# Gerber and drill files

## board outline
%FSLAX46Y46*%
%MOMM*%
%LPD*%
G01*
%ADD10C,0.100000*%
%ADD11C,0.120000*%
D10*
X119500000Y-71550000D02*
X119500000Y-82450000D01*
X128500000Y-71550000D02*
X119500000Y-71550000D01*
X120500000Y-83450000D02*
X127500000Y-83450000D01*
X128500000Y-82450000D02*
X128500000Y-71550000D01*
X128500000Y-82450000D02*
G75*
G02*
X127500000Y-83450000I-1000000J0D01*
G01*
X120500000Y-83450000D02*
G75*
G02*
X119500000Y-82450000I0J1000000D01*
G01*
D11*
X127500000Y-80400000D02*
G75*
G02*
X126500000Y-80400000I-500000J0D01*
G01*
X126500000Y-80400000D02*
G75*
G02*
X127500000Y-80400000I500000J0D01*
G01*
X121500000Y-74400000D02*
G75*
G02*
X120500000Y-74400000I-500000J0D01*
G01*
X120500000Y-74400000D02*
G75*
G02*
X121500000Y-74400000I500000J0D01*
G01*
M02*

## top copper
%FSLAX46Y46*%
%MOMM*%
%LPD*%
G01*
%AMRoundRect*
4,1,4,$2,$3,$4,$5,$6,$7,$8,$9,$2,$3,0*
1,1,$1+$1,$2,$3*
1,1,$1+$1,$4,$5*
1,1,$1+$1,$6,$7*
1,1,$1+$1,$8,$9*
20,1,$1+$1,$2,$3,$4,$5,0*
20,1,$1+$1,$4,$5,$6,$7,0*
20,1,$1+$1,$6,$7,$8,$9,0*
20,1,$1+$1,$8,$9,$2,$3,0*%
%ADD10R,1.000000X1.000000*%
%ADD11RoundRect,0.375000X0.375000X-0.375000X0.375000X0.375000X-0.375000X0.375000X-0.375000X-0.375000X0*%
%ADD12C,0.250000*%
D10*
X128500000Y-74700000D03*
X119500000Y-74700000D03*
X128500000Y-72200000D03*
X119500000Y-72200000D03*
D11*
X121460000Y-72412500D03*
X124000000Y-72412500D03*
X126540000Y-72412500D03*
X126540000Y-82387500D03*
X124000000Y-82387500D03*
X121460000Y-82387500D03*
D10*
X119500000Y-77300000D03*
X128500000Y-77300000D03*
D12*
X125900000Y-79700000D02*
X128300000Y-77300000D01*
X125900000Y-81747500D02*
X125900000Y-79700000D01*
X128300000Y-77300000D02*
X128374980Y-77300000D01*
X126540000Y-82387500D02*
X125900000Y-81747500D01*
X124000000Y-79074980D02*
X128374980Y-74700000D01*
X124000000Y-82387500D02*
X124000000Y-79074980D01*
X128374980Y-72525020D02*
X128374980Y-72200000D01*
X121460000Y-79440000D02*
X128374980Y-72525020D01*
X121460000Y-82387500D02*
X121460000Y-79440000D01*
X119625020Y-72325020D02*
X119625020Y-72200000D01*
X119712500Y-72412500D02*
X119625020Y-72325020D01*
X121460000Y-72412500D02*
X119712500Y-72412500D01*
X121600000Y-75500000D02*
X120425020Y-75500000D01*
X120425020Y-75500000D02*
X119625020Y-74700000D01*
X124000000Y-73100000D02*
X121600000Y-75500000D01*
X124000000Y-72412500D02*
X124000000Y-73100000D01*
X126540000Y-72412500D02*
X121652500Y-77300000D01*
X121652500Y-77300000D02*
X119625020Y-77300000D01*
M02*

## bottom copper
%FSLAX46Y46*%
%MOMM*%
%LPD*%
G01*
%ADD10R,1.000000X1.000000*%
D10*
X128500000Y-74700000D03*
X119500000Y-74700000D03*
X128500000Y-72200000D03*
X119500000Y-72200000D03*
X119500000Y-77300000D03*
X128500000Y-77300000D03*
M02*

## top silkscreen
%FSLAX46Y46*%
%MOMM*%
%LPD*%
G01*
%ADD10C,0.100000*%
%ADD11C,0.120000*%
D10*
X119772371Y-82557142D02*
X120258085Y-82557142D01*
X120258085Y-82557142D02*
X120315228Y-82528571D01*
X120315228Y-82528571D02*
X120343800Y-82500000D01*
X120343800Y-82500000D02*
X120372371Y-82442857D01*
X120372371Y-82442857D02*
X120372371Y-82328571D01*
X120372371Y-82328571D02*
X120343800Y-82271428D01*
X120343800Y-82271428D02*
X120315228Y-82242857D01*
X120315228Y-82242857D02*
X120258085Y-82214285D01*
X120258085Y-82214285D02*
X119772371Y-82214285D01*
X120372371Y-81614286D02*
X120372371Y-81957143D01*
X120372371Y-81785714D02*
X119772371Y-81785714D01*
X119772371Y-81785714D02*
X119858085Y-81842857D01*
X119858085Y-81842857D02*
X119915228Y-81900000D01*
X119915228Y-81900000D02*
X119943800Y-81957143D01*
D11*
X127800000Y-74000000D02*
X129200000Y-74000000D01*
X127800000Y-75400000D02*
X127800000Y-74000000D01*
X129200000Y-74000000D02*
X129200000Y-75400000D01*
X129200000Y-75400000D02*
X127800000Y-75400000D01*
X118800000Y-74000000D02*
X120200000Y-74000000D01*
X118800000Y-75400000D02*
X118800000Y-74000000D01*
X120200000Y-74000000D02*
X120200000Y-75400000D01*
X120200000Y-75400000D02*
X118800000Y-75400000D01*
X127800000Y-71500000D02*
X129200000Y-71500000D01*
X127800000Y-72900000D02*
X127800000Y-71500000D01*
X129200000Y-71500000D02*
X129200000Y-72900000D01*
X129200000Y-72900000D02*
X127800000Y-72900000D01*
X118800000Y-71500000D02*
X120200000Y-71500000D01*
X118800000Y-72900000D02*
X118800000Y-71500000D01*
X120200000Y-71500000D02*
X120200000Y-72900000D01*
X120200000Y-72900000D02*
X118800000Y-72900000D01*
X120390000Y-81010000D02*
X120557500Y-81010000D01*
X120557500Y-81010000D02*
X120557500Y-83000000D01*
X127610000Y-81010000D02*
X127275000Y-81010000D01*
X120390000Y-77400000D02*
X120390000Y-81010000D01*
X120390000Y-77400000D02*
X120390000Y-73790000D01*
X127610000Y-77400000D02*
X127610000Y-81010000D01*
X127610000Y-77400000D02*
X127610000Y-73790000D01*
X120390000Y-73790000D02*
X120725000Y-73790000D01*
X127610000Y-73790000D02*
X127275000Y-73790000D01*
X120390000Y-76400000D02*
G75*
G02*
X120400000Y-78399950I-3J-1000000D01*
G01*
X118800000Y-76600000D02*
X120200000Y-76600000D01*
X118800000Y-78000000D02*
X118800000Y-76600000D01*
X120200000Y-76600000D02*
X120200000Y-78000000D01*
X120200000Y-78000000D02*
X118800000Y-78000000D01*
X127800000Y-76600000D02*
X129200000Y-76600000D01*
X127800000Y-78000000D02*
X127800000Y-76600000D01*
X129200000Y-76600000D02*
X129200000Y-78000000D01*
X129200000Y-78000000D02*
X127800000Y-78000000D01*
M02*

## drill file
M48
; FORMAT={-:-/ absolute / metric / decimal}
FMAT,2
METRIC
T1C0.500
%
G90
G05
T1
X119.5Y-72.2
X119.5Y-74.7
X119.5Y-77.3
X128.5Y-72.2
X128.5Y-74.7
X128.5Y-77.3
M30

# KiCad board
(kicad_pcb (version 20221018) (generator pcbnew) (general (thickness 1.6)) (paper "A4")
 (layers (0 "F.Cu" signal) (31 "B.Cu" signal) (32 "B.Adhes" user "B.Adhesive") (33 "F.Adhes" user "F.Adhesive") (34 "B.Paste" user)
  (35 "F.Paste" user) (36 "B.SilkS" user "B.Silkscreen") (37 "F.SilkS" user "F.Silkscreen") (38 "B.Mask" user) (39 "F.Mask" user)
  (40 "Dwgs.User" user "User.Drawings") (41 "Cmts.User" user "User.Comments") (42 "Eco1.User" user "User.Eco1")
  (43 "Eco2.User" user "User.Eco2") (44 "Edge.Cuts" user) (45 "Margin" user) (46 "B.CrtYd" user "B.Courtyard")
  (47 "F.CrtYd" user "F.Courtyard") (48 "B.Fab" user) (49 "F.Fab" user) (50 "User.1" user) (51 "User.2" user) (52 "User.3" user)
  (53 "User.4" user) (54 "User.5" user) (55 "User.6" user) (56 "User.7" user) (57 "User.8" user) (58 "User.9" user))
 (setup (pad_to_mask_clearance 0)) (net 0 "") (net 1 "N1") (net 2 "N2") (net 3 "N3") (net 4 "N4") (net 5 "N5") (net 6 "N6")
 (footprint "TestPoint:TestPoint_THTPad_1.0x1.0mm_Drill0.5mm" (layer "F.Cu") (at 128.5 74.7)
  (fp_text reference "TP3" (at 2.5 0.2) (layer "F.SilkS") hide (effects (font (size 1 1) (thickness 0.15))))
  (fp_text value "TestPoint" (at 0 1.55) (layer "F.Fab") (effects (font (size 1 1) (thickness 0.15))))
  (fp_line (start -0.7 -0.7) (end 0.7 -0.7) (stroke (width 0.12) (type solid)) (layer "F.SilkS"))
  (fp_line (start -0.7 0.7) (end -0.7 -0.7) (stroke (width 0.12) (type solid)) (layer "F.SilkS"))
  (fp_line (start 0.7 -0.7) (end 0.7 0.7) (stroke (width 0.12) (type solid)) (layer "F.SilkS"))
  (fp_line (start 0.7 0.7) (end -0.7 0.7) (stroke (width 0.12) (type solid)) (layer "F.SilkS"))
  (pad "1" thru_hole rect (at 0 0) (size 1 1) (drill 0.5) (layers "*.Cu" "*.Mask") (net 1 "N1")))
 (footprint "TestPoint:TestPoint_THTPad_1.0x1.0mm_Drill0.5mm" (layer "F.Cu") (at 119.5 74.7)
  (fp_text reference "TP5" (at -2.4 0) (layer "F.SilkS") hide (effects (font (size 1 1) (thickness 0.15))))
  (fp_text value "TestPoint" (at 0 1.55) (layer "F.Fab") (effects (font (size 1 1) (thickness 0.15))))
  (fp_line (start -0.7 -0.7) (end 0.7 -0.7) (stroke (width 0.12) (type solid)) (layer "F.SilkS"))
  (fp_line (start -0.7 0.7) (end -0.7 -0.7) (stroke (width 0.12) (type solid)) (layer "F.SilkS"))
  (fp_line (start 0.7 -0.7) (end 0.7 0.7) (stroke (width 0.12) (type solid)) (layer "F.SilkS"))
  (fp_line (start 0.7 0.7) (end -0.7 0.7) (stroke (width 0.12) (type solid)) (layer "F.SilkS"))
  (pad "1" thru_hole rect (at 0 0) (size 1 1) (drill 0.5) (layers "*.Cu" "*.Mask") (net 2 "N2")))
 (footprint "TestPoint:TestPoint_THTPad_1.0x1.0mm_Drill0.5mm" (layer "F.Cu") (at 128.5 72.2)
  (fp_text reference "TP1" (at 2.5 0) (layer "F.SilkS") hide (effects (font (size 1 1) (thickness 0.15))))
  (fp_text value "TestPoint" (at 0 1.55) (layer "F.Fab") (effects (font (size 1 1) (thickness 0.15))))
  (fp_line (start -0.7 -0.7) (end 0.7 -0.7) (stroke (width 0.12) (type solid)) (layer "F.SilkS"))
  (fp_line (start -0.7 0.7) (end -0.7 -0.7) (stroke (width 0.12) (type solid)) (layer "F.SilkS"))
  (fp_line (start 0.7 -0.7) (end 0.7 0.7) (stroke (width 0.12) (type solid)) (layer "F.SilkS"))
  (fp_line (start 0.7 0.7) (end -0.7 0.7) (stroke (width 0.12) (type solid)) (layer "F.SilkS"))
  (pad "1" thru_hole rect (at 0 0) (size 1 1) (drill 0.5) (layers "*.Cu" "*.Mask") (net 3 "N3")))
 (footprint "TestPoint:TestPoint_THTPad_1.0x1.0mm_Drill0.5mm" (layer "F.Cu") (at 119.5 72.2)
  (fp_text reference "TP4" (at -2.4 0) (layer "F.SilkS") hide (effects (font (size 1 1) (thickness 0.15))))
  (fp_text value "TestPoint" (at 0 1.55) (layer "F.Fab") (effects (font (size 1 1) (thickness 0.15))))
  (fp_line (start -0.7 -0.7) (end 0.7 -0.7) (stroke (width 0.12) (type solid)) (layer "F.SilkS"))
  (fp_line (start -0.7 0.7) (end -0.7 -0.7) (stroke (width 0.12) (type solid)) (layer "F.SilkS"))
  (fp_line (start 0.7 -0.7) (end 0.7 0.7) (stroke (width 0.12) (type solid)) (layer "F.SilkS"))
  (fp_line (start 0.7 0.7) (end -0.7 0.7) (stroke (width 0.12) (type solid)) (layer "F.SilkS"))
  (pad "1" thru_hole rect (at 0 0) (size 1 1) (drill 0.5) (layers "*.Cu" "*.Mask") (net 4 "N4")))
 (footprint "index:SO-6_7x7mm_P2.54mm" (layer "F.Cu") (at 124 77.4 90)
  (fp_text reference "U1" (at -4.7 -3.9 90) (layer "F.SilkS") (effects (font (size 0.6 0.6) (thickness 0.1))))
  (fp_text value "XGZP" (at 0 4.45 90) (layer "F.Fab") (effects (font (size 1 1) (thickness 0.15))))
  (fp_line (start -3.61 -3.61) (end -3.61 -3.4425) (stroke (width 0.12) (type solid)) (layer "F.SilkS"))
  (fp_line (start -3.61 -3.4425) (end -5.6 -3.4425) (stroke (width 0.12) (type solid)) (layer "F.SilkS"))
  (fp_line (start -3.61 3.61) (end -3.61 3.275) (stroke (width 0.12) (type solid)) (layer "F.SilkS"))
  (fp_line (start 0 -3.61) (end -3.61 -3.61) (stroke (width 0.12) (type solid)) (layer "F.SilkS"))
  (fp_line (start 0 -3.61) (end 3.61 -3.61) (stroke (width 0.12) (type solid)) (layer "F.SilkS"))
  (fp_line (start 0 3.61) (end -3.61 3.61) (stroke (width 0.12) (type solid)) (layer "F.SilkS"))
  (fp_line (start 0 3.61) (end 3.61 3.61) (stroke (width 0.12) (type solid)) (layer "F.SilkS"))
  (fp_line (start 3.61 -3.61) (end 3.61 -3.275) (stroke (width 0.12) (type solid)) (layer "F.SilkS"))
  (fp_line (start 3.61 3.61) (end 3.61 3.275) (stroke (width 0.12) (type solid)) (layer "F.SilkS"))
  (fp_arc (start 1 -3.61) (mid 0.005 -2.610015) (end -0.99995 -3.6) (stroke (width 0.12) (type solid)) (layer "F.SilkS"))
  (fp_circle (center -3 3) (end -2.5 3) (stroke (width 0.12) (type solid)) (fill none) (layer "Edge.Cuts"))
  (fp_circle (center 3 -3) (end 3.5 -3) (stroke (width 0.12) (type solid)) (fill none) (layer "Edge.Cuts"))
  (pad "1" smd roundrect (at 4.9875 -2.54 90) (size 1.5 1.5) (layers "F.Cu" "F.Paste" "F.Mask") (roundrect_rratio 0.25) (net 4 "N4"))
  (pad "2" smd roundrect (at 4.9875 0 90) (size 1.5 1.5) (layers "F.Cu" "F.Paste" "F.Mask") (roundrect_rratio 0.25) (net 2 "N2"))
  (pad "3" smd roundrect (at 4.9875 2.54 90) (size 1.5 1.5) (layers "F.Cu" "F.Paste" "F.Mask") (roundrect_rratio 0.25) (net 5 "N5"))
  (pad "4" smd roundrect (at -4.9875 2.54 90) (size 1.5 1.5) (layers "F.Cu" "F.Paste" "F.Mask") (roundrect_rratio 0.25) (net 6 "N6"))
  (pad "5" smd roundrect (at -4.9875 0 90) (size 1.5 1.5) (layers "F.Cu" "F.Paste" "F.Mask") (roundrect_rratio 0.25) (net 1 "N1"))
  (pad "6" smd roundrect (at -4.9875 -2.54 90) (size 1.5 1.5) (layers "F.Cu" "F.Paste" "F.Mask") (roundrect_rratio 0.25) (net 3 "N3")))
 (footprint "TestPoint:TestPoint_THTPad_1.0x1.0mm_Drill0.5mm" (layer "F.Cu") (at 119.5 77.3)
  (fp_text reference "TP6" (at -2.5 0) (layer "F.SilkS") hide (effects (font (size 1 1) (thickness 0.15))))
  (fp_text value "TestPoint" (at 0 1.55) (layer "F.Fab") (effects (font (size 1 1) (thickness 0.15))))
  (fp_line (start -0.7 -0.7) (end 0.7 -0.7) (stroke (width 0.12) (type solid)) (layer "F.SilkS"))
  (fp_line (start -0.7 0.7) (end -0.7 -0.7) (stroke (width 0.12) (type solid)) (layer "F.SilkS"))
  (fp_line (start 0.7 -0.7) (end 0.7 0.7) (stroke (width 0.12) (type solid)) (layer "F.SilkS"))
  (fp_line (start 0.7 0.7) (end -0.7 0.7) (stroke (width 0.12) (type solid)) (layer "F.SilkS"))
  (pad "1" thru_hole rect (at 0 0) (size 1 1) (drill 0.5) (layers "*.Cu" "*.Mask") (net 5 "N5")))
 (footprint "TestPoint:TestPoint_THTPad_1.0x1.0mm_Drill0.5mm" (layer "F.Cu") (at 128.5 77.3)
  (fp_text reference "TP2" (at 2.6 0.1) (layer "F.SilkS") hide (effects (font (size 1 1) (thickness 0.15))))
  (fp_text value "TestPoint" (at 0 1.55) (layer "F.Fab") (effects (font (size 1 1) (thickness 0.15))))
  (fp_line (start -0.7 -0.7) (end 0.7 -0.7) (stroke (width 0.12) (type solid)) (layer "F.SilkS"))
  (fp_line (start -0.7 0.7) (end -0.7 -0.7) (stroke (width 0.12) (type solid)) (layer "F.SilkS"))
  (fp_line (start 0.7 -0.7) (end 0.7 0.7) (stroke (width 0.12) (type solid)) (layer "F.SilkS"))
  (fp_line (start 0.7 0.7) (end -0.7 0.7) (stroke (width 0.12) (type solid)) (layer "F.SilkS"))
  (pad "1" thru_hole rect (at 0 0) (size 1 1) (drill 0.5) (layers "*.Cu" "*.Mask") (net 6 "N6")))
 (gr_line (start 119.5 71.55) (end 119.5 82.45) (stroke (width 0.1) (type solid)) (layer "Edge.Cuts"))
 (gr_line (start 128.5 71.55) (end 119.5 71.55) (stroke (width 0.1) (type solid)) (layer "Edge.Cuts"))
 (gr_line (start 120.5 83.45) (end 127.5 83.45) (stroke (width 0.1) (type solid)) (layer "Edge.Cuts"))
 (gr_line (start 128.5 82.45) (end 128.5 71.55) (stroke (width 0.1) (type solid)) (layer "Edge.Cuts"))
 (gr_arc (start 128.5 82.45) (mid 128.207107 83.157107) (end 127.5 83.45) (stroke (width 0.1) (type solid)) (layer "Edge.Cuts"))
 (gr_arc (start 120.5 83.45) (mid 119.792893 83.157107) (end 119.5 82.45) (stroke (width 0.1) (type solid)) (layer "Edge.Cuts"))
 (segment (start 125.9 79.7) (end 128.3 77.3) (width 0.25) (layer "F.Cu") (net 6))
 (segment (start 125.9 81.7475) (end 125.9 79.7) (width 0.25) (layer "F.Cu") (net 6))
 (segment (start 128.3 77.3) (end 128.37498 77.3) (width 0.25) (layer "F.Cu") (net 6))
 (segment (start 126.54 82.3875) (end 125.9 81.7475) (width 0.25) (layer "F.Cu") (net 6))
 (segment (start 124 79.07498) (end 128.37498 74.7) (width 0.25) (layer "F.Cu") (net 1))
 (segment (start 124 82.3875) (end 124 79.07498) (width 0.25) (layer "F.Cu") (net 1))
 (segment (start 128.37498 72.52502) (end 128.37498 72.2) (width 0.25) (layer "F.Cu") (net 3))
 (segment (start 121.46 79.44) (end 128.37498 72.52502) (width 0.25) (layer "F.Cu") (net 3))
 (segment (start 121.46 82.3875) (end 121.46 79.44) (width 0.25) (layer "F.Cu") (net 3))
 (segment (start 119.62502 72.32502) (end 119.62502 72.2) (width 0.25) (layer "F.Cu") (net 4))
 (segment (start 119.7125 72.4125) (end 119.62502 72.32502) (width 0.25) (layer "F.Cu") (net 4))
 (segment (start 121.46 72.4125) (end 119.7125 72.4125) (width 0.25) (layer "F.Cu") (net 4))
 (segment (start 121.6 75.5) (end 120.42502 75.5) (width 0.25) (layer "F.Cu") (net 2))
 (segment (start 120.42502 75.5) (end 119.62502 74.7) (width 0.25) (layer "F.Cu") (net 2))
 (segment (start 124 73.1) (end 121.6 75.5) (width 0.25) (layer "F.Cu") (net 2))
 (segment (start 124 72.4125) (end 124 73.1) (width 0.25) (layer "F.Cu") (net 2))
 (segment (start 126.54 72.4125) (end 121.6525 77.3) (width 0.25) (layer "F.Cu") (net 5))
 (segment (start 121.6525 77.3) (end 119.62502 77.3) (width 0.25) (layer "F.Cu") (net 5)))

